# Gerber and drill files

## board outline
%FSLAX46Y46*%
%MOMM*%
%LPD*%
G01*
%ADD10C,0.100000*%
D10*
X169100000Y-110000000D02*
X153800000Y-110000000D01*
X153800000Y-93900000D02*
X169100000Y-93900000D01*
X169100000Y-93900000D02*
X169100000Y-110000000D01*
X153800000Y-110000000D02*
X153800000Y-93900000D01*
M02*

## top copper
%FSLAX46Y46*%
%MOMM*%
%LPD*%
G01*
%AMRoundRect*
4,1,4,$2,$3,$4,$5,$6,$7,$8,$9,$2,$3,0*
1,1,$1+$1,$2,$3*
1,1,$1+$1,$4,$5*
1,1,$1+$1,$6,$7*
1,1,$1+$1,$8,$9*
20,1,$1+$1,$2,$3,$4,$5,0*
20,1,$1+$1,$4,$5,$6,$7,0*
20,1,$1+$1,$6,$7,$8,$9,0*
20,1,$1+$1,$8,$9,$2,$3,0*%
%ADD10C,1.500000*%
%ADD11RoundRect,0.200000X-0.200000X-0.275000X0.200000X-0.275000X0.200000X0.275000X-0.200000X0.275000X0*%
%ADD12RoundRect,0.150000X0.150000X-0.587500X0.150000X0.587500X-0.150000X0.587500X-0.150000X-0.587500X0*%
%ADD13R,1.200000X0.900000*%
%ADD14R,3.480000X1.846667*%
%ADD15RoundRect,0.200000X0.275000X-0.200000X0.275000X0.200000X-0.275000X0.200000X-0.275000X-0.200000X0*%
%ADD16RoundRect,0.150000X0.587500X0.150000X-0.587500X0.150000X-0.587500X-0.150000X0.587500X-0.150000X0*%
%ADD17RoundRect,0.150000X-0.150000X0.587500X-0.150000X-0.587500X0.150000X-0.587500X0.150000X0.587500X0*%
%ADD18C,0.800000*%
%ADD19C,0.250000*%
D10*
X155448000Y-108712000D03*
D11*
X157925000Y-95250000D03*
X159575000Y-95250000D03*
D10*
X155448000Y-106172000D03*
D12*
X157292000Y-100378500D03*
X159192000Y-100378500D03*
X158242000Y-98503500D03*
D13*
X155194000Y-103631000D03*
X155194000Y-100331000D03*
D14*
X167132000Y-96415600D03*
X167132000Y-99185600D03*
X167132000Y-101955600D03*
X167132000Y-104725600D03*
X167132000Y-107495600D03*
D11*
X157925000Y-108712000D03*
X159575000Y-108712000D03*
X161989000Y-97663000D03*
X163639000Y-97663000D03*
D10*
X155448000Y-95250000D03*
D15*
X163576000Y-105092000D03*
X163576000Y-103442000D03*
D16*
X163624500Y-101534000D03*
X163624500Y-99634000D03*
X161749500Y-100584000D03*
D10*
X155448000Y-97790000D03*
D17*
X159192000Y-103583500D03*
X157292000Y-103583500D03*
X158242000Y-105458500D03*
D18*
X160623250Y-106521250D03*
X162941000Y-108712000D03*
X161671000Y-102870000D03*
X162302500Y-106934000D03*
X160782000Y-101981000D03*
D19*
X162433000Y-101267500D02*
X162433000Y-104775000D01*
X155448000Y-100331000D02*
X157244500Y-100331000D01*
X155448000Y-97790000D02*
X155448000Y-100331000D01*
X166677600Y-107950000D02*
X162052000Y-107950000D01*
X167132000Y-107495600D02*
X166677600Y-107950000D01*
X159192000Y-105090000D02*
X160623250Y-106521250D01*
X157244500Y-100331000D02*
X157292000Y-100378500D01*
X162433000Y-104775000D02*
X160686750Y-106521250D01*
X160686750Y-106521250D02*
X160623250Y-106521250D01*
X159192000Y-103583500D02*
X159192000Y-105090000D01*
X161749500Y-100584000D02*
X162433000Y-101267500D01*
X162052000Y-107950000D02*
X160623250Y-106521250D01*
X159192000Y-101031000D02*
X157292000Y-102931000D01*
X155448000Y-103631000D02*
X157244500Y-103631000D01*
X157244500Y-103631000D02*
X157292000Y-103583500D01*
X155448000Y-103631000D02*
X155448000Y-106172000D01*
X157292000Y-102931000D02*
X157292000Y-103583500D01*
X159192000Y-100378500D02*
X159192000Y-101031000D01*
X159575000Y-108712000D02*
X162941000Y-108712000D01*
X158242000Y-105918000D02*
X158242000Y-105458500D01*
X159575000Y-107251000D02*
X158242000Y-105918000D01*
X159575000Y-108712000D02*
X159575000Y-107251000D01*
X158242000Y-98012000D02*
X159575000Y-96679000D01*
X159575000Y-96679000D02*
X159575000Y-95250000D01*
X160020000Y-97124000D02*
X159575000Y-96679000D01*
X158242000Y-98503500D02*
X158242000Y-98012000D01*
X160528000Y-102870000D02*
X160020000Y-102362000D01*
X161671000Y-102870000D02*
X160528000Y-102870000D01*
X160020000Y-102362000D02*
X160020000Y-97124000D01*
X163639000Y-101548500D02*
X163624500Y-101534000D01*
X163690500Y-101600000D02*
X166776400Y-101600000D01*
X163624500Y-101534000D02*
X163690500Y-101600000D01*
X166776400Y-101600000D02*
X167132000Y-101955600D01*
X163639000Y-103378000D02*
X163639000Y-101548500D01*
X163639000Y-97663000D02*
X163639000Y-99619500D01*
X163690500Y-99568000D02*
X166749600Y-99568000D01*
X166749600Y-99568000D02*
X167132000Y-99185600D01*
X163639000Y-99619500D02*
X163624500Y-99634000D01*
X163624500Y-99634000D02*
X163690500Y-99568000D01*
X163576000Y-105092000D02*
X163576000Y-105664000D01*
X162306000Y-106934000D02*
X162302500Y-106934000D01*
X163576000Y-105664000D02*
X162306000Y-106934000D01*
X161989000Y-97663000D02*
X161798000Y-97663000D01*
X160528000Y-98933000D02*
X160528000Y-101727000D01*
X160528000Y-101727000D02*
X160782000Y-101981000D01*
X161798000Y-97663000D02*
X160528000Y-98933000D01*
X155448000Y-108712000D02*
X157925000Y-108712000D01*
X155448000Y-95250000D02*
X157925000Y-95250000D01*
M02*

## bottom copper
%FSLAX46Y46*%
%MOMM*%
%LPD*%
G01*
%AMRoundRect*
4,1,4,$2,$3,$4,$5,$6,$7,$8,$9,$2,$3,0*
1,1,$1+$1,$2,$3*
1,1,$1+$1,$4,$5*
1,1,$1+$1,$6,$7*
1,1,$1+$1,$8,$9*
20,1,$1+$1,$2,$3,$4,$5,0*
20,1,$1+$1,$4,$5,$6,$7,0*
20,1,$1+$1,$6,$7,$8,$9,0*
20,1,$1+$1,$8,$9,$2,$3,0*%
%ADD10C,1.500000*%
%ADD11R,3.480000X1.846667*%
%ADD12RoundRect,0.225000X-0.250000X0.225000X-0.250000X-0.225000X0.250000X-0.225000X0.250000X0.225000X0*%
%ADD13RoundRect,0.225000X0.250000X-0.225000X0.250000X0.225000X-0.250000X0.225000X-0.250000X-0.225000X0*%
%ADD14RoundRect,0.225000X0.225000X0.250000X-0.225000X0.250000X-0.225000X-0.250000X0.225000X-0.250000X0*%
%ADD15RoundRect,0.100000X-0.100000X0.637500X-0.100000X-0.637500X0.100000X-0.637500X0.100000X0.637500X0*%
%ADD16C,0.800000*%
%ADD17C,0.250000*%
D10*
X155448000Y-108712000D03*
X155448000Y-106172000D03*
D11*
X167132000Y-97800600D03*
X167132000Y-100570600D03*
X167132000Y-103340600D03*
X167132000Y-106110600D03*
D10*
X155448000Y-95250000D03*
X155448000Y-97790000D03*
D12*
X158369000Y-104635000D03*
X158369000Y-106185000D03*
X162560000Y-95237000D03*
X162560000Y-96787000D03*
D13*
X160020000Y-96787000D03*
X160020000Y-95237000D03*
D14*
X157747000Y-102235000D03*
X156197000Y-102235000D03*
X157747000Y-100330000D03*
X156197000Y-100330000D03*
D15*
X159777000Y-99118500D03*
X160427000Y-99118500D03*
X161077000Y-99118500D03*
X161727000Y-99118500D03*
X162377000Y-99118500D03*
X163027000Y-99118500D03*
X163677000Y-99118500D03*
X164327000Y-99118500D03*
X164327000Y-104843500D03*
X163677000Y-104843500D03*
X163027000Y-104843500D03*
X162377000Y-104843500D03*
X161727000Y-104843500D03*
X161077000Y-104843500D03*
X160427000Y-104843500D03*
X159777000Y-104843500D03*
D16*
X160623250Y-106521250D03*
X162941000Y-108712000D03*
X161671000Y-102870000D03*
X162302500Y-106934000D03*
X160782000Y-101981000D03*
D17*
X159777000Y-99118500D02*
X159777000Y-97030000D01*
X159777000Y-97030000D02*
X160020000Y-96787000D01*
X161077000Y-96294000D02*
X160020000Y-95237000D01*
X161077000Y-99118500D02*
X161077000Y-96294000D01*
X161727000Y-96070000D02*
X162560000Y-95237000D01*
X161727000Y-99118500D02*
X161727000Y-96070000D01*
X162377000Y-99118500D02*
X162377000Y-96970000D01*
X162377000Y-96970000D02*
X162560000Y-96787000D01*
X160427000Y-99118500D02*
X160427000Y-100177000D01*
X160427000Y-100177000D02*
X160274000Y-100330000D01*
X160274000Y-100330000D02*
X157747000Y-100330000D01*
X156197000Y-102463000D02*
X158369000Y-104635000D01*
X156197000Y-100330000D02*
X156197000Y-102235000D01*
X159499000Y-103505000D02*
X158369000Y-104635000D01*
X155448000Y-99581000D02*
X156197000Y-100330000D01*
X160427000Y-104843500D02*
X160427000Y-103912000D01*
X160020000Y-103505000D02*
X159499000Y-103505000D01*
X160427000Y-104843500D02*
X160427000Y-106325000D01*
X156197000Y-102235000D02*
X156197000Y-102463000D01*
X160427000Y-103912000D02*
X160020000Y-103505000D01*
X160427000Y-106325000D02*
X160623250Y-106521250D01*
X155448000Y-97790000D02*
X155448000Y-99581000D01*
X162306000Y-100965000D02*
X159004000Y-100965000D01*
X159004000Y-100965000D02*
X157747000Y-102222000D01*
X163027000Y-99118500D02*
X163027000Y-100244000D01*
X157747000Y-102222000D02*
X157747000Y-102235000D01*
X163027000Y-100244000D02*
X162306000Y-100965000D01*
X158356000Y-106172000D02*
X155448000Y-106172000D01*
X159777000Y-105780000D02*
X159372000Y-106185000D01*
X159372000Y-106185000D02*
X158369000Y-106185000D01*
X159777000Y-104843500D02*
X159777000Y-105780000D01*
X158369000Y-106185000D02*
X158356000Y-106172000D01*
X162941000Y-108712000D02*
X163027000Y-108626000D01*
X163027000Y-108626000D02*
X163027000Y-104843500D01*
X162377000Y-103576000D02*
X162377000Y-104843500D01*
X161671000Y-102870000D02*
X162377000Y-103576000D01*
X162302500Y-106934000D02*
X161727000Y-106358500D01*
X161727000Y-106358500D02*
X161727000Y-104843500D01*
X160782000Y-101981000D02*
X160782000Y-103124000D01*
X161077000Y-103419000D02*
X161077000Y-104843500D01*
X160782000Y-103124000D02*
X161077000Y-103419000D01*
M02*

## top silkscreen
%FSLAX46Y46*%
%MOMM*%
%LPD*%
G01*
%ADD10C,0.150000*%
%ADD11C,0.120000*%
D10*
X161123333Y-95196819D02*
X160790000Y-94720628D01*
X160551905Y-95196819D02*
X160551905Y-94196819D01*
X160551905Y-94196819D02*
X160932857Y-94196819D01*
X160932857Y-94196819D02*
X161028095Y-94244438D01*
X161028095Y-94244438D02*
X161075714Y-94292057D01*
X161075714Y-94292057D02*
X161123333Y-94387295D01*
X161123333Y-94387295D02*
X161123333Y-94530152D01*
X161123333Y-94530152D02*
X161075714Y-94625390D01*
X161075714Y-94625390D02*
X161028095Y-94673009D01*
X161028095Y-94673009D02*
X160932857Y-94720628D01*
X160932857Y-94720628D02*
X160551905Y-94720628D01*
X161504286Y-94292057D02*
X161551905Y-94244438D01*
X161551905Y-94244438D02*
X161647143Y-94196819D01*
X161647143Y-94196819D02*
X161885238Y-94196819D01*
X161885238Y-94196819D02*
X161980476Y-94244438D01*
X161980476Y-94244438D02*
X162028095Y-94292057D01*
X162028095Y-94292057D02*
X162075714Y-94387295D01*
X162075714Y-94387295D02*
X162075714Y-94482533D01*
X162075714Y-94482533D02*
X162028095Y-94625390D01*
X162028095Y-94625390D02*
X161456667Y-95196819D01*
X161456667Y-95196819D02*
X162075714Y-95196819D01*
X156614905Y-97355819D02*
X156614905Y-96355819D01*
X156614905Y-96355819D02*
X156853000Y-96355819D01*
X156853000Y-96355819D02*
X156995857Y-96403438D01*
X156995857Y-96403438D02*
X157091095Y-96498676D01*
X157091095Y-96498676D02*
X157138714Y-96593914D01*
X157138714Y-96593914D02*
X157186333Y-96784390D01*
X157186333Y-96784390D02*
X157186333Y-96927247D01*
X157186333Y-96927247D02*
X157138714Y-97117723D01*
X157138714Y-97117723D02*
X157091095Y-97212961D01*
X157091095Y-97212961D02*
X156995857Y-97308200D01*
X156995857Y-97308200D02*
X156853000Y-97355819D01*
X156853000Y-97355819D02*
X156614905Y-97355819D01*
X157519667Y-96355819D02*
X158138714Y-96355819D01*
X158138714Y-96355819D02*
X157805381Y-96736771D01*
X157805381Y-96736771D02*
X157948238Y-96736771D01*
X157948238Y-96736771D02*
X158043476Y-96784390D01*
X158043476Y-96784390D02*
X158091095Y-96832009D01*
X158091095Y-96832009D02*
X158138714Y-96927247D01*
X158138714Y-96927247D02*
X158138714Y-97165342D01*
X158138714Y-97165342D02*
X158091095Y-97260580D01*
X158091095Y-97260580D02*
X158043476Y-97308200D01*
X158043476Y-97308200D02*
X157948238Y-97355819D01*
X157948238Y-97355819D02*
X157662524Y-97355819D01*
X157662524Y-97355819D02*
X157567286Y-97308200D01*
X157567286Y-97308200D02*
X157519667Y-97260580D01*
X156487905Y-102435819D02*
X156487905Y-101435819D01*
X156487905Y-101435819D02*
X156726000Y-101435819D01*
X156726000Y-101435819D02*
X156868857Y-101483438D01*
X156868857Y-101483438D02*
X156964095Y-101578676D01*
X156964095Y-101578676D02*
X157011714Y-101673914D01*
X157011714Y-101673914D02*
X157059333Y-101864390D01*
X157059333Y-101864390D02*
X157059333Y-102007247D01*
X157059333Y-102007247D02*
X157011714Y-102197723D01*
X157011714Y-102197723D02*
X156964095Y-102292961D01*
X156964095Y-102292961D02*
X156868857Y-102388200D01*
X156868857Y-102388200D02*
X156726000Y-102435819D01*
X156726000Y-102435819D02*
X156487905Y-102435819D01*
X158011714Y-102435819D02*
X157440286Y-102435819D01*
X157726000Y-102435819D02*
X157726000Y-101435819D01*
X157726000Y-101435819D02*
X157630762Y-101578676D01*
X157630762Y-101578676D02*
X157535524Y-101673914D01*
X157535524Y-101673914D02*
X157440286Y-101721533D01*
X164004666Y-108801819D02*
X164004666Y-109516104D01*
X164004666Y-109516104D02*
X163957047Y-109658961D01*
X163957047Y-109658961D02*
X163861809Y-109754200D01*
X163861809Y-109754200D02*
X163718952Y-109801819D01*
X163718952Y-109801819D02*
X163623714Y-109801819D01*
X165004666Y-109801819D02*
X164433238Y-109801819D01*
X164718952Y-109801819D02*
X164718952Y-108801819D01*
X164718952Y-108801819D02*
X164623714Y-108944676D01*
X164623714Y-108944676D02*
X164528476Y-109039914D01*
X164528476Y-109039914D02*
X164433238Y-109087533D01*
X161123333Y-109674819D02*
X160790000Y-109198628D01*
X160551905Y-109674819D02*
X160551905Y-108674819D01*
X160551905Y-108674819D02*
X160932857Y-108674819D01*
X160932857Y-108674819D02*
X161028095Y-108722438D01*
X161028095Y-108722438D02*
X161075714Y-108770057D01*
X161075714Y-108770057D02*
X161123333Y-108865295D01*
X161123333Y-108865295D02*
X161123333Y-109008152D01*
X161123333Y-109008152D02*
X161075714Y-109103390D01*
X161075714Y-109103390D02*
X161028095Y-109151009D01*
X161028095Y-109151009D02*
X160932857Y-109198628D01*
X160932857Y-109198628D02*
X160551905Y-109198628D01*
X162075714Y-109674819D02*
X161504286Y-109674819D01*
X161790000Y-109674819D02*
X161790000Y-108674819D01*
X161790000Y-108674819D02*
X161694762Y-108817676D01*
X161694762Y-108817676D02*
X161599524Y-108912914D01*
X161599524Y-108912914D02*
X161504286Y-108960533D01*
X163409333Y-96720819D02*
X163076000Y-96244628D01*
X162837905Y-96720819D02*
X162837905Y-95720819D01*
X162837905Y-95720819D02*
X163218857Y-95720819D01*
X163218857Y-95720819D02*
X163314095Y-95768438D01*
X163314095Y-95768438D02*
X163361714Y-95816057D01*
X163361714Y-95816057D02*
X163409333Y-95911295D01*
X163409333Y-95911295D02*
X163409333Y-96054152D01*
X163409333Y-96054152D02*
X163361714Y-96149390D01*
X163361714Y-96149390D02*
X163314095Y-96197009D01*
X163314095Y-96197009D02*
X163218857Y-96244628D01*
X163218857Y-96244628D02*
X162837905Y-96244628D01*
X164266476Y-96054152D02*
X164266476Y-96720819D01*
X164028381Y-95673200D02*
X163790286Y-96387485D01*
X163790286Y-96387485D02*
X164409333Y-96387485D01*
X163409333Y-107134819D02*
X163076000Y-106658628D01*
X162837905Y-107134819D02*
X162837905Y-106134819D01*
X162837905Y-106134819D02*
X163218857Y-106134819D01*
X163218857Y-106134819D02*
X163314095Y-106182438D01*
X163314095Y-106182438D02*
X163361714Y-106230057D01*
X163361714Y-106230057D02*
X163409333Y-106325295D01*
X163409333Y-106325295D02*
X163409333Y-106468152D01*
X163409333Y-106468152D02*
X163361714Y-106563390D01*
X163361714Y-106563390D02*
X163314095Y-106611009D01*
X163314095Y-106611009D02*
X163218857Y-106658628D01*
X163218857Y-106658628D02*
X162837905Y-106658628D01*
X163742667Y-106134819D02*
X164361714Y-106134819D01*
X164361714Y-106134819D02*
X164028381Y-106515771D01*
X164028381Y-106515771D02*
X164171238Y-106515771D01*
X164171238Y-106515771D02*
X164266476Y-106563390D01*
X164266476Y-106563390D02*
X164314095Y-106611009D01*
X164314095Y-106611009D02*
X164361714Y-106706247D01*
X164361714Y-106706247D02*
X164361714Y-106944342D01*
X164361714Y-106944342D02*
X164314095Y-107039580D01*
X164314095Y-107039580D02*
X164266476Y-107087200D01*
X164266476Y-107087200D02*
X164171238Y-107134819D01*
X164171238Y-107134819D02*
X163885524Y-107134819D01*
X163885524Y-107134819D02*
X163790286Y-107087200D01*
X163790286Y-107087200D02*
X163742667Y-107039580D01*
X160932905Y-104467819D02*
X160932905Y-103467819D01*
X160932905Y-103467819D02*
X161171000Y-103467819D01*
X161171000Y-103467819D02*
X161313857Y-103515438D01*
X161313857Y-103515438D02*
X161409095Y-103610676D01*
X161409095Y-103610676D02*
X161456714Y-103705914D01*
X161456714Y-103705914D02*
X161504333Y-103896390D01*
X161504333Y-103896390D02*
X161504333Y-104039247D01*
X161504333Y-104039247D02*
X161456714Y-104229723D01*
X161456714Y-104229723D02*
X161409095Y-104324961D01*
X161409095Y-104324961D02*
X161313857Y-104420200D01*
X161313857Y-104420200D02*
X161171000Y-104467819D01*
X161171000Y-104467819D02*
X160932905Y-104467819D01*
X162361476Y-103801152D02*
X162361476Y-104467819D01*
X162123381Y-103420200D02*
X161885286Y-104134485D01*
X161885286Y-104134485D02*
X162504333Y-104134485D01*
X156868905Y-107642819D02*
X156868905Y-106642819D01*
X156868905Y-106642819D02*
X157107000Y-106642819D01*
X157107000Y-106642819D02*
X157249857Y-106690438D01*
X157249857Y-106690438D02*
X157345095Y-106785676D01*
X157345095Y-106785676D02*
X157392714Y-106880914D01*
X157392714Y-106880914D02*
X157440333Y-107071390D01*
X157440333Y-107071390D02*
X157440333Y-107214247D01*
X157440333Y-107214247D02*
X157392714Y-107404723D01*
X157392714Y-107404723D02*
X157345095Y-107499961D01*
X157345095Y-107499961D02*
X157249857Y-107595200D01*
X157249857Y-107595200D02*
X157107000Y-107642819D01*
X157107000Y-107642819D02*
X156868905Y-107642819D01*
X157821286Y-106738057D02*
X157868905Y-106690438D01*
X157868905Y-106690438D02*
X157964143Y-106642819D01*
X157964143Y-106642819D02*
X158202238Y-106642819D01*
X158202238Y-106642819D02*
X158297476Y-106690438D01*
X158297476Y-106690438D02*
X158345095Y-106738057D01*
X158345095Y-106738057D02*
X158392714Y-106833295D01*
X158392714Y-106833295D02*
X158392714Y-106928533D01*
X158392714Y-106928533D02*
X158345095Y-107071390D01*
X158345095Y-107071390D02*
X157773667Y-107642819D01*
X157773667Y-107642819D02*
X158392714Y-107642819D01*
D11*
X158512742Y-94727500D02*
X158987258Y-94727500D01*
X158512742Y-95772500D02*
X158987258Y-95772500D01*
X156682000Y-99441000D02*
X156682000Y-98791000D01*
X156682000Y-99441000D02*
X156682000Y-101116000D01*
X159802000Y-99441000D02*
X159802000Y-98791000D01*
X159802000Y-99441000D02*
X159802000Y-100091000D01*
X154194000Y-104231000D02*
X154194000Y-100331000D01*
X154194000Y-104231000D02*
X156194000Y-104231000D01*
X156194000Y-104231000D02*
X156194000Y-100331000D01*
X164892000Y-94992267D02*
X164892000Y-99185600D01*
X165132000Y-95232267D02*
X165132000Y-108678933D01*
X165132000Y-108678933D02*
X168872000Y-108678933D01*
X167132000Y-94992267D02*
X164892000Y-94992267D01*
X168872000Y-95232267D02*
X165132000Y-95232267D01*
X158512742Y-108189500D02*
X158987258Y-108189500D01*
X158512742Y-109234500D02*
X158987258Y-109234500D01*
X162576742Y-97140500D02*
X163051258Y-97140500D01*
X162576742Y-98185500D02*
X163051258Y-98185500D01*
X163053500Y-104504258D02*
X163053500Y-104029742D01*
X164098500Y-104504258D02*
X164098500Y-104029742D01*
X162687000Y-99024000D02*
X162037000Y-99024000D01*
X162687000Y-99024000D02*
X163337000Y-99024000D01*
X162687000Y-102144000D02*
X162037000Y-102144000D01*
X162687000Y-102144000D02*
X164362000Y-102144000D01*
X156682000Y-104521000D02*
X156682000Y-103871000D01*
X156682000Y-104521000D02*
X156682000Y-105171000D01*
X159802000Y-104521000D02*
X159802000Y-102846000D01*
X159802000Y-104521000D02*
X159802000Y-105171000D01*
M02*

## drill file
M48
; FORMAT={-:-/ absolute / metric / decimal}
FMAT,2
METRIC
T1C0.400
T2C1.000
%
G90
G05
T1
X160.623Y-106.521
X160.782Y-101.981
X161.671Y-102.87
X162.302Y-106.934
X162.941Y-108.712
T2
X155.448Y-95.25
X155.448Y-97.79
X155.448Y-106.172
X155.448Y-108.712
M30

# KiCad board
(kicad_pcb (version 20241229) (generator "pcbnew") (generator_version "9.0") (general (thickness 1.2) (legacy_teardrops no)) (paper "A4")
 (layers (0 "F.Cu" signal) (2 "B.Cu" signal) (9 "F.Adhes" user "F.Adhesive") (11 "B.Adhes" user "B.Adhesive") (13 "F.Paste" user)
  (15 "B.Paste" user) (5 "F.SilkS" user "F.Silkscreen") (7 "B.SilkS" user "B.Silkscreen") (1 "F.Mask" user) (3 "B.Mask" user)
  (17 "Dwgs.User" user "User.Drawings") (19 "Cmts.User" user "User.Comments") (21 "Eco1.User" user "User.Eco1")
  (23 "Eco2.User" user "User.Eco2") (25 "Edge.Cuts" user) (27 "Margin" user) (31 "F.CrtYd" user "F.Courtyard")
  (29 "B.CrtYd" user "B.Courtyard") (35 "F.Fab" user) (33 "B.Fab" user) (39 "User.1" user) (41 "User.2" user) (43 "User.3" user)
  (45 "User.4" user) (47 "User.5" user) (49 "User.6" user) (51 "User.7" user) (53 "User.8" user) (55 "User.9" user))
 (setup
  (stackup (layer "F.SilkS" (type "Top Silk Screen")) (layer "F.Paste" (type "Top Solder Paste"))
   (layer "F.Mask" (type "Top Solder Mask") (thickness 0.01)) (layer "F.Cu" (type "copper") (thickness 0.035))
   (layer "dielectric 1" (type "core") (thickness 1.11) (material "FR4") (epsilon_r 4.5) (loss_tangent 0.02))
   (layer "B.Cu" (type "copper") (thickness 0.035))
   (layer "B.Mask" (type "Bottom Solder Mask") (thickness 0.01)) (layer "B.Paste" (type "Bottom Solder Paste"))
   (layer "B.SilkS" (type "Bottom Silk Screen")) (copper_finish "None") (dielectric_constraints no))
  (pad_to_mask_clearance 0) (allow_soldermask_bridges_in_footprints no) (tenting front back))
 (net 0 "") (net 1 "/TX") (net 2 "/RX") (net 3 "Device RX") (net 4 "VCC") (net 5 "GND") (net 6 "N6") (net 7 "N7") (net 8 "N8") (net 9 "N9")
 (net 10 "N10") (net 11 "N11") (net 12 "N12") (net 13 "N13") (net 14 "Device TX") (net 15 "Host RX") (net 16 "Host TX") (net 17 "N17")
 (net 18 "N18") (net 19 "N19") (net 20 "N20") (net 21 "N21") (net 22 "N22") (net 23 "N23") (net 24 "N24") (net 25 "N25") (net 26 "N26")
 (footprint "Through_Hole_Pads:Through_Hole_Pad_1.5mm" (layer "F.Cu") (at 155.448 108.712)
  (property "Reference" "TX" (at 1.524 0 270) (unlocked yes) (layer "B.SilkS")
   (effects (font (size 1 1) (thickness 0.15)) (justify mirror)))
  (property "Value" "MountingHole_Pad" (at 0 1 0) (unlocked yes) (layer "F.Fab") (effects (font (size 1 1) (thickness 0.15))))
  (pad "1" thru_hole circle (at 0 0) (size 1.5 1.5) (drill 1) (layers "*.Cu" "*.Mask") (remove_unused_layers no) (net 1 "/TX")))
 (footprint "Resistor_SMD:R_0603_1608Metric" (layer "F.Cu") (at 158.75 95.25)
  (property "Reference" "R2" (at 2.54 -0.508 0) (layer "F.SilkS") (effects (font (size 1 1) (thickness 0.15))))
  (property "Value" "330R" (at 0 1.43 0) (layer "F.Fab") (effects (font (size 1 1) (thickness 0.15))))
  (fp_line (start -0.237258 -0.5225) (end 0.237258 -0.5225) (stroke (width 0.12) (type solid)) (layer "F.SilkS"))
  (fp_line (start -0.237258 0.5225) (end 0.237258 0.5225) (stroke (width 0.12) (type solid)) (layer "F.SilkS"))
  (pad "1" smd roundrect (at -0.825 0) (size 0.8 0.95) (layers "F.Cu" "F.Mask" "F.Paste") (roundrect_rratio 0.25) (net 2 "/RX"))
  (pad "2" smd roundrect (at 0.825 0) (size 0.8 0.95) (layers "F.Cu" "F.Mask" "F.Paste") (roundrect_rratio 0.25) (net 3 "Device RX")))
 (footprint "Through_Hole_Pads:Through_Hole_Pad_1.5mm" (layer "F.Cu") (at 155.448 106.172)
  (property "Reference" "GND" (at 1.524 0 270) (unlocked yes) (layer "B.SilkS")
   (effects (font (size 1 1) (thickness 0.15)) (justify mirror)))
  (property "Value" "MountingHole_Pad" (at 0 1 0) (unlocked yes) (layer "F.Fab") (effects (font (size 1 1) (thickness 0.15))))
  (pad "1" thru_hole circle (at 0 0) (size 1.5 1.5) (drill 1) (layers "*.Cu" "*.Mask") (remove_unused_layers no) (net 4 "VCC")))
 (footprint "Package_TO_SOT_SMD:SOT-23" (layer "F.Cu") (at 158.242 99.441 90)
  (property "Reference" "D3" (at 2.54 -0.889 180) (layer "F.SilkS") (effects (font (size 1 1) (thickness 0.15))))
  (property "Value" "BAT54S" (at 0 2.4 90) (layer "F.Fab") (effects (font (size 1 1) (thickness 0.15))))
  (fp_line (start 0 -1.56) (end 0.65 -1.56) (stroke (width 0.12) (type solid)) (layer "F.SilkS"))
  (fp_line (start 0 -1.56) (end -1.675 -1.56) (stroke (width 0.12) (type solid)) (layer "F.SilkS"))
  (fp_line (start 0 1.56) (end 0.65 1.56) (stroke (width 0.12) (type solid)) (layer "F.SilkS"))
  (fp_line (start 0 1.56) (end -0.65 1.56) (stroke (width 0.12) (type solid)) (layer "F.SilkS"))
  (pad "1" smd roundrect (at -0.9375 -0.95 90) (size 1.475 0.6) (layers "F.Cu" "F.Mask" "F.Paste") (roundrect_rratio 0.25) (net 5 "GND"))
  (pad "2" smd roundrect (at -0.9375 0.95 90) (size 1.475 0.6) (layers "F.Cu" "F.Mask" "F.Paste") (roundrect_rratio 0.25) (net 4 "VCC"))
  (pad "3" smd roundrect (at 0.9375 0 90) (size 1.475 0.6) (layers "F.Cu" "F.Mask" "F.Paste") (roundrect_rratio 0.25) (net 3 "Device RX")))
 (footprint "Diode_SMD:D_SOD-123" (layer "F.Cu") (at 155.194 101.981 90)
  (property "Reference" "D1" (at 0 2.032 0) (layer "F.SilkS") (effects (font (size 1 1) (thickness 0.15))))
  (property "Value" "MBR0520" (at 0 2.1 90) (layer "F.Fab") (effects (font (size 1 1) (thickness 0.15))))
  (fp_line (start -2.25 -1) (end 1.65 -1) (stroke (width 0.12) (type solid)) (layer "F.SilkS"))
  (fp_line (start -2.25 -1) (end -2.25 1) (stroke (width 0.12) (type solid)) (layer "F.SilkS"))
  (fp_line (start -2.25 1) (end 1.65 1) (stroke (width 0.12) (type solid)) (layer "F.SilkS"))
  (pad "1" smd rect (at -1.65 0 90) (size 0.9 1.2) (layers "F.Cu" "F.Mask" "F.Paste") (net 4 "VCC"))
  (pad "2" smd rect (at 1.65 0 90) (size 0.9 1.2) (layers "F.Cu" "F.Mask" "F.Paste") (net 5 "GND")))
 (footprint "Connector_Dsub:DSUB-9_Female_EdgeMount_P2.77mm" (layer "F.Cu") (at 167.132 101.9556 90)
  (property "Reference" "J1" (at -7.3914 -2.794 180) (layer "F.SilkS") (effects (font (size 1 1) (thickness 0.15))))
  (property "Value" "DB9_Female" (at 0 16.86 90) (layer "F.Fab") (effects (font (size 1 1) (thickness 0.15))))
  (fp_line (start 6.963333 -2.24) (end 2.77 -2.24) (stroke (width 0.12) (type solid)) (layer "F.SilkS"))
  (fp_line (start 6.723333 -2) (end -6.723333 -2) (stroke (width 0.12) (type solid)) (layer "F.SilkS"))
  (fp_line (start -6.723333 -2) (end -6.723333 1.74) (stroke (width 0.12) (type solid)) (layer "F.SilkS"))
  (fp_line (start 6.963333 0) (end 6.963333 -2.24) (stroke (width 0.12) (type solid)) (layer "F.SilkS"))
  (fp_line (start 6.723333 1.74) (end 6.723333 -2) (stroke (width 0.12) (type solid)) (layer "F.SilkS"))
  (pad "1" smd rect (at 5.54 0 90) (size 1.846667 3.48) (layers "F.Cu" "F.Mask" "F.Paste") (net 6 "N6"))
  (pad "2" smd rect (at 2.77 0 90) (size 1.846667 3.48) (layers "F.Cu" "F.Mask" "F.Paste") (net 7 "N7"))
  (pad "3" smd rect (at 0 0 90) (size 1.846667 3.48) (layers "F.Cu" "F.Mask" "F.Paste") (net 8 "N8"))
  (pad "4" smd rect (at -2.77 0 90) (size 1.846667 3.48) (layers "F.Cu" "F.Mask" "F.Paste") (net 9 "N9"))
  (pad "5" smd rect (at -5.54 0 90) (size 1.846667 3.48) (layers "F.Cu" "F.Mask" "F.Paste") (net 5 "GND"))
  (pad "6" smd rect (at 4.155 0 90) (size 1.846667 3.48) (layers "B.Cu" "B.Mask" "B.Paste") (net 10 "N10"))
  (pad "7" smd rect (at 1.385 0 90) (size 1.846667 3.48) (layers "B.Cu" "B.Mask" "B.Paste") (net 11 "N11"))
  (pad "8" smd rect (at -1.385 0 90) (size 1.846667 3.48) (layers "B.Cu" "B.Mask" "B.Paste") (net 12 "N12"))
  (pad "9" smd rect (at -4.155 0 90) (size 1.846667 3.48) (layers "B.Cu" "B.Mask" "B.Paste") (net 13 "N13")))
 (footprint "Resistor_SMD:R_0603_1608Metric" (layer "F.Cu") (at 158.75 108.712)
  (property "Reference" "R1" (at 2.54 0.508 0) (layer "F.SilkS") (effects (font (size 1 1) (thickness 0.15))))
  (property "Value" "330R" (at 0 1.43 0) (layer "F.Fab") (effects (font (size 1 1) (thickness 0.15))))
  (fp_line (start -0.237258 -0.5225) (end 0.237258 -0.5225) (stroke (width 0.12) (type solid)) (layer "F.SilkS"))
  (fp_line (start -0.237258 0.5225) (end 0.237258 0.5225) (stroke (width 0.12) (type solid)) (layer "F.SilkS"))
  (pad "1" smd roundrect (at -0.825 0) (size 0.8 0.95) (layers "F.Cu" "F.Mask" "F.Paste") (roundrect_rratio 0.25) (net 1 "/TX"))
  (pad "2" smd roundrect (at 0.825 0) (size 0.8 0.95) (layers "F.Cu" "F.Mask" "F.Paste") (roundrect_rratio 0.25) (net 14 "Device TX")))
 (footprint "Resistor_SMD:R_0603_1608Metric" (layer "F.Cu") (at 162.814 97.663)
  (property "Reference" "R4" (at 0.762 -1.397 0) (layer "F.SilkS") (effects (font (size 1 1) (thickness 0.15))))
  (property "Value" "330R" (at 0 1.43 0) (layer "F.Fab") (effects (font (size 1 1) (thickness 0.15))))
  (fp_line (start -0.237258 -0.5225) (end 0.237258 -0.5225) (stroke (width 0.12) (type solid)) (layer "F.SilkS"))
  (fp_line (start -0.237258 0.5225) (end 0.237258 0.5225) (stroke (width 0.12) (type solid)) (layer "F.SilkS"))
  (pad "1" smd roundrect (at -0.825 0) (size 0.8 0.95) (layers "F.Cu" "F.Mask" "F.Paste") (roundrect_rratio 0.25) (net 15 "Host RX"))
  (pad "2" smd roundrect (at 0.825 0) (size 0.8 0.95) (layers "F.Cu" "F.Mask" "F.Paste") (roundrect_rratio 0.25) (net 7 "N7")))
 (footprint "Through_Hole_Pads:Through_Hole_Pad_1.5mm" (layer "F.Cu") (at 155.448 95.25)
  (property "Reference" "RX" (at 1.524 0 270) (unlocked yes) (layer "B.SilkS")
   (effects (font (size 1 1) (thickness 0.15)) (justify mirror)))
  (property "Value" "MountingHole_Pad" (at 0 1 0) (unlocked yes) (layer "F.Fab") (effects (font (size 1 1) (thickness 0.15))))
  (pad "1" thru_hole circle (at 0 0) (size 1.5 1.5) (drill 1) (layers "*.Cu" "*.Mask") (remove_unused_layers no) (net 2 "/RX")))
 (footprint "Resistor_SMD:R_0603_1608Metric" (layer "F.Cu") (at 163.576 104.267 90)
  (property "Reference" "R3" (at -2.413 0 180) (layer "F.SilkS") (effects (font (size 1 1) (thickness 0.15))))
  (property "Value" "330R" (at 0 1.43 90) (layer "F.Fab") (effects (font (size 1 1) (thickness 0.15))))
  (fp_line (start -0.237258 -0.5225) (end 0.237258 -0.5225) (stroke (width 0.12) (type solid)) (layer "F.SilkS"))
  (fp_line (start -0.237258 0.5225) (end 0.237258 0.5225) (stroke (width 0.12) (type solid)) (layer "F.SilkS"))
  (pad "1" smd roundrect (at -0.825 0 90) (size 0.8 0.95) (layers "F.Cu" "F.Mask" "F.Paste") (roundrect_rratio 0.25) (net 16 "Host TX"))
  (pad "2" smd roundrect (at 0.825 0 90) (size 0.8 0.95) (layers "F.Cu" "F.Mask" "F.Paste") (roundrect_rratio 0.25) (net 8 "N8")))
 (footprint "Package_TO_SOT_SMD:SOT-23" (layer "F.Cu") (at 162.687 100.584 180)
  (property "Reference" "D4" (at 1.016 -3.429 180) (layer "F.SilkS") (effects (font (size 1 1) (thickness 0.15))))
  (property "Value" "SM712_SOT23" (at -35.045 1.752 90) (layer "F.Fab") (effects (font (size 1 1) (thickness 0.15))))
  (fp_line (start 0 1.56) (end 0.65 1.56) (stroke (width 0.12) (type solid)) (layer "F.SilkS"))
  (fp_line (start 0 1.56) (end -0.65 1.56) (stroke (width 0.12) (type solid)) (layer "F.SilkS"))
  (fp_line (start 0 -1.56) (end 0.65 -1.56) (stroke (width 0.12) (type solid)) (layer "F.SilkS"))
  (fp_line (start 0 -1.56) (end -1.675 -1.56) (stroke (width 0.12) (type solid)) (layer "F.SilkS"))
  (pad "1" smd roundrect (at -0.9375 -0.95 180) (size 1.475 0.6) (layers "F.Cu" "F.Mask" "F.Paste") (roundrect_rratio 0.25) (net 8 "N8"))
  (pad "2" smd roundrect (at -0.9375 0.95 180) (size 1.475 0.6) (layers "F.Cu" "F.Mask" "F.Paste") (roundrect_rratio 0.25) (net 7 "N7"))
  (pad "3" smd roundrect (at 0.9375 0 180) (size 1.475 0.6) (layers "F.Cu" "F.Mask" "F.Paste") (roundrect_rratio 0.25) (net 5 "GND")))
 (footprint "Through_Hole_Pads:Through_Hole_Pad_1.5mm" (layer "F.Cu") (at 155.448 97.79 180)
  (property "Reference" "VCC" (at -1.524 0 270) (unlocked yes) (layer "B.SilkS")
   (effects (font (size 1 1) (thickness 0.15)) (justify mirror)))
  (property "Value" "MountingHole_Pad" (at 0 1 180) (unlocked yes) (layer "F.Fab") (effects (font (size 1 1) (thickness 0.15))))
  (pad "1" thru_hole circle (at 0 0 180) (size 1.5 1.5) (drill 1) (layers "*.Cu" "*.Mask") (remove_unused_layers no) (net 5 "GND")))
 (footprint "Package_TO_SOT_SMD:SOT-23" (layer "F.Cu") (at 158.242 104.521 -90)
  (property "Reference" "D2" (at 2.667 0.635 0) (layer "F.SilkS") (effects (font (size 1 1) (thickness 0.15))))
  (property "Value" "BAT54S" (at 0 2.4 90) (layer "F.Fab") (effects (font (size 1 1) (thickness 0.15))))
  (fp_line (start 0 1.56) (end -0.65 1.56) (stroke (width 0.12) (type solid)) (layer "F.SilkS"))
  (fp_line (start 0 1.56) (end 0.65 1.56) (stroke (width 0.12) (type solid)) (layer "F.SilkS"))
  (fp_line (start 0 -1.56) (end -1.675 -1.56) (stroke (width 0.12) (type solid)) (layer "F.SilkS"))
  (fp_line (start 0 -1.56) (end 0.65 -1.56) (stroke (width 0.12) (type solid)) (layer "F.SilkS"))
  (pad "1" smd roundrect (at -0.9375 -0.95 270) (size 1.475 0.6) (layers "F.Cu" "F.Mask" "F.Paste") (roundrect_rratio 0.25) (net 5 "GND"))
  (pad "2" smd roundrect (at -0.9375 0.95 270) (size 1.475 0.6) (layers "F.Cu" "F.Mask" "F.Paste") (roundrect_rratio 0.25) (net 4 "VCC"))
  (pad "3" smd roundrect (at 0.9375 0 270) (size 1.475 0.6) (layers "F.Cu" "F.Mask" "F.Paste") (roundrect_rratio 0.25) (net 14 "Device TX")))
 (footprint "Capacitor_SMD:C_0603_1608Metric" (layer "B.Cu") (at 158.369 105.41 -90)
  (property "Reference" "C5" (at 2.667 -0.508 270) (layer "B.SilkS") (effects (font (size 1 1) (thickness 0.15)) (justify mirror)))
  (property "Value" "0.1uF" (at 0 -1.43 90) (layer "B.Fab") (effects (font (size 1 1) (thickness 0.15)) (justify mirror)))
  (pad "1" smd roundrect (at -0.775 0 270) (size 0.9 0.95) (layers "B.Cu" "B.Mask" "B.Paste") (roundrect_rratio 0.25) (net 5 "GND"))
  (pad "2" smd roundrect (at 0.775 0 270) (size 0.9 0.95) (layers "B.Cu" "B.Mask" "B.Paste") (roundrect_rratio 0.25) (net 4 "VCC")))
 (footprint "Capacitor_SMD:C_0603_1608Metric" (layer "B.Cu") (at 162.56 96.012 -90)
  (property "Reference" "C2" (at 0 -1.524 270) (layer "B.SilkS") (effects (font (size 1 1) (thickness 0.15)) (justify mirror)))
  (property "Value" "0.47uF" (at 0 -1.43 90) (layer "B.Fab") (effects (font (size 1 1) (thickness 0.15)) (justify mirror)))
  (pad "1" smd roundrect (at -0.775 0 270) (size 0.9 0.95) (layers "B.Cu" "B.Mask" "B.Paste") (roundrect_rratio 0.25) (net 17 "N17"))
  (pad "2" smd roundrect (at 0.775 0 270) (size 0.9 0.95) (layers "B.Cu" "B.Mask" "B.Paste") (roundrect_rratio 0.25) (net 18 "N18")))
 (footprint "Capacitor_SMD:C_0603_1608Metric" (layer "B.Cu") (at 160.02 96.012 90)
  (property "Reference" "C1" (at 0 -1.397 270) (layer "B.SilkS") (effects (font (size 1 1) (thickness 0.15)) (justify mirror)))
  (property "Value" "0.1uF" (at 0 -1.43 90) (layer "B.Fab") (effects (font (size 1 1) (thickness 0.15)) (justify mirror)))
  (pad "1" smd roundrect (at -0.775 0 90) (size 0.9 0.95) (layers "B.Cu" "B.Mask" "B.Paste") (roundrect_rratio 0.25) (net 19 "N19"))
  (pad "2" smd roundrect (at 0.775 0 90) (size 0.9 0.95) (layers "B.Cu" "B.Mask" "B.Paste") (roundrect_rratio 0.25) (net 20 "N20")))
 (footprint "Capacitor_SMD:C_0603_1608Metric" (layer "B.Cu") (at 156.972 102.235 180)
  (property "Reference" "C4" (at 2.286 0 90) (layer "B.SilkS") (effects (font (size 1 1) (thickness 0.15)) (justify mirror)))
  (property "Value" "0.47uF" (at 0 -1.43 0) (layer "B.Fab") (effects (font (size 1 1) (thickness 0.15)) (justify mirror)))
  (pad "1" smd roundrect (at -0.775 0 180) (size 0.9 0.95) (layers "B.Cu" "B.Mask" "B.Paste") (roundrect_rratio 0.25) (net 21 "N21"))
  (pad "2" smd roundrect (at 0.775 0 180) (size 0.9 0.95) (layers "B.Cu" "B.Mask" "B.Paste") (roundrect_rratio 0.25) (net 5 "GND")))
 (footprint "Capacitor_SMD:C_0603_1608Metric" (layer "B.Cu") (at 156.972 100.33 180)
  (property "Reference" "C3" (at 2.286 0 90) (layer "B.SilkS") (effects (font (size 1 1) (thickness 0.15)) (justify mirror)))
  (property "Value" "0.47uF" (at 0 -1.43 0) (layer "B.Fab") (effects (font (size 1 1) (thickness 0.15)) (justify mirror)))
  (pad "1" smd roundrect (at -0.775 0 180) (size 0.9 0.95) (layers "B.Cu" "B.Mask" "B.Paste") (roundrect_rratio 0.25) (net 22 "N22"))
  (pad "2" smd roundrect (at 0.775 0 180) (size 0.9 0.95) (layers "B.Cu" "B.Mask" "B.Paste") (roundrect_rratio 0.25) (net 5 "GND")))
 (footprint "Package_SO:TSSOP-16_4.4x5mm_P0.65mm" (layer "B.Cu") (at 162.052 101.981 -90)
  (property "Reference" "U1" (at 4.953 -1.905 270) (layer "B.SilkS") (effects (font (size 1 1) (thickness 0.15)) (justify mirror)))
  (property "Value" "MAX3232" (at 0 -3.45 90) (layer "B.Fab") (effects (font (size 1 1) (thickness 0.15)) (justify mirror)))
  (pad "1" smd roundrect (at -2.8625 2.275 270) (size 1.475 0.4) (layers "B.Cu" "B.Mask" "B.Paste") (roundrect_rratio 0.25) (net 19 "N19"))
  (pad "2" smd roundrect (at -2.8625 1.625 270) (size 1.475 0.4) (layers "B.Cu" "B.Mask" "B.Paste") (roundrect_rratio 0.25) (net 22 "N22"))
  (pad "3" smd roundrect (at -2.8625 0.975 270) (size 1.475 0.4) (layers "B.Cu" "B.Mask" "B.Paste") (roundrect_rratio 0.25) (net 20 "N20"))
  (pad "4" smd roundrect (at -2.8625 0.325 270) (size 1.475 0.4) (layers "B.Cu" "B.Mask" "B.Paste") (roundrect_rratio 0.25) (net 17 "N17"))
  (pad "5" smd roundrect (at -2.8625 -0.325 270) (size 1.475 0.4) (layers "B.Cu" "B.Mask" "B.Paste") (roundrect_rratio 0.25) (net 18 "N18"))
  (pad "6" smd roundrect (at -2.8625 -0.975 270) (size 1.475 0.4) (layers "B.Cu" "B.Mask" "B.Paste") (roundrect_rratio 0.25) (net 21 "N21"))
  (pad "7" smd roundrect (at -2.8625 -1.625 270) (size 1.475 0.4) (layers "B.Cu" "B.Mask" "B.Paste") (roundrect_rratio 0.25) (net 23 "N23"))
  (pad "8" smd roundrect (at -2.8625 -2.275 270) (size 1.475 0.4) (layers "B.Cu" "B.Mask" "B.Paste") (roundrect_rratio 0.25) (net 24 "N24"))
  (pad "9" smd roundrect (at 2.8625 -2.275 270) (size 1.475 0.4) (layers "B.Cu" "B.Mask" "B.Paste") (roundrect_rratio 0.25) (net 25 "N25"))
  (pad "10" smd roundrect (at 2.8625 -1.625 270) (size 1.475 0.4) (layers "B.Cu" "B.Mask" "B.Paste") (roundrect_rratio 0.25) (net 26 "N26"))
  (pad "11" smd roundrect (at 2.8625 -0.975 270) (size 1.475 0.4) (layers "B.Cu" "B.Mask" "B.Paste") (roundrect_rratio 0.25)
   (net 14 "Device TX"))
  (pad "12" smd roundrect (at 2.8625 -0.325 270) (size 1.475 0.4) (layers "B.Cu" "B.Mask" "B.Paste") (roundrect_rratio 0.25)
   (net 3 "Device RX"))
  (pad "13" smd roundrect (at 2.8625 0.325 270) (size 1.475 0.4) (layers "B.Cu" "B.Mask" "B.Paste") (roundrect_rratio 0.25)
   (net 16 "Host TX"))
  (pad "14" smd roundrect (at 2.8625 0.975 270) (size 1.475 0.4) (layers "B.Cu" "B.Mask" "B.Paste") (roundrect_rratio 0.25)
   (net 15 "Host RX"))
  (pad "15" smd roundrect (at 2.8625 1.625 270) (size 1.475 0.4) (layers "B.Cu" "B.Mask" "B.Paste") (roundrect_rratio 0.25) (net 5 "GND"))
  (pad "16" smd roundrect (at 2.8625 2.275 270) (size 1.475 0.4) (layers "B.Cu" "B.Mask" "B.Paste") (roundrect_rratio 0.25) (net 4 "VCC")))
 (gr_line (start 169.1 110) (end 153.8 110) (stroke (width 0.1) (type solid)) (layer "Edge.Cuts"))
 (gr_line (start 153.8 93.9) (end 169.1 93.9) (stroke (width 0.1) (type solid)) (layer "Edge.Cuts"))
 (gr_line (start 169.1 93.9) (end 169.1 110) (stroke (width 0.1) (type solid)) (layer "Edge.Cuts"))
 (gr_line (start 153.8 110) (end 153.8 93.9) (stroke (width 0.1) (type solid)) (layer "Edge.Cuts"))
 (segment (start 159.777 99.1185) (end 159.777 97.03) (width 0.25) (layer "B.Cu") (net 19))
 (segment (start 159.777 97.03) (end 160.02 96.787) (width 0.25) (layer "B.Cu") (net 19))
 (segment (start 161.077 96.294) (end 160.02 95.237) (width 0.25) (layer "B.Cu") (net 20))
 (segment (start 161.077 99.1185) (end 161.077 96.294) (width 0.25) (layer "B.Cu") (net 20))
 (segment (start 161.727 96.07) (end 162.56 95.237) (width 0.25) (layer "B.Cu") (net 17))
 (segment (start 161.727 99.1185) (end 161.727 96.07) (width 0.25) (layer "B.Cu") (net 17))
 (segment (start 162.377 99.1185) (end 162.377 96.97) (width 0.25) (layer "B.Cu") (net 18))
 (segment (start 162.377 96.97) (end 162.56 96.787) (width 0.25) (layer "B.Cu") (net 18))
 (segment (start 160.427 99.1185) (end 160.427 100.177) (width 0.25) (layer "B.Cu") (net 22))
 (segment (start 160.427 100.177) (end 160.274 100.33) (width 0.25) (layer "B.Cu") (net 22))
 (segment (start 160.274 100.33) (end 157.747 100.33) (width 0.25) (layer "B.Cu") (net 22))
 (segment (start 162.433 101.2675) (end 162.433 104.775) (width 0.25) (layer "F.Cu") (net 5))
 (segment (start 155.448 100.331) (end 157.2445 100.331) (width 0.25) (layer "F.Cu") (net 5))
 (segment (start 155.448 97.79) (end 155.448 100.331) (width 0.25) (layer "F.Cu") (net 5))
 (segment (start 166.6776 107.95) (end 162.052 107.95) (width 0.25) (layer "F.Cu") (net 5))
 (segment (start 167.132 107.4956) (end 166.6776 107.95) (width 0.25) (layer "F.Cu") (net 5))
 (segment (start 159.192 105.09) (end 160.62325 106.52125) (width 0.25) (layer "F.Cu") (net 5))
 (segment (start 157.2445 100.331) (end 157.292 100.3785) (width 0.25) (layer "F.Cu") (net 5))
 (segment (start 162.433 104.775) (end 160.68675 106.52125) (width 0.25) (layer "F.Cu") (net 5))
 (segment (start 160.68675 106.52125) (end 160.62325 106.52125) (width 0.25) (layer "F.Cu") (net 5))
 (segment (start 159.192 103.5835) (end 159.192 105.09) (width 0.25) (layer "F.Cu") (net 5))
 (segment (start 161.7495 100.584) (end 162.433 101.2675) (width 0.25) (layer "F.Cu") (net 5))
 (segment (start 162.052 107.95) (end 160.62325 106.52125) (width 0.25) (layer "F.Cu") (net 5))
 (via (at 160.62325 106.52125) (size 0.8) (drill 0.4) (layers "F.Cu" "B.Cu") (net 5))
 (segment (start 156.197 102.463) (end 158.369 104.635) (width 0.25) (layer "B.Cu") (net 5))
 (segment (start 156.197 100.33) (end 156.197 102.235) (width 0.25) (layer "B.Cu") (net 5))
 (segment (start 159.499 103.505) (end 158.369 104.635) (width 0.25) (layer "B.Cu") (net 5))
 (segment (start 155.448 99.581) (end 156.197 100.33) (width 0.25) (layer "B.Cu") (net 5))
 (segment (start 160.427 104.8435) (end 160.427 103.912) (width 0.25) (layer "B.Cu") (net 5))
 (segment (start 160.02 103.505) (end 159.499 103.505) (width 0.25) (layer "B.Cu") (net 5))
 (segment (start 160.427 104.8435) (end 160.427 106.325) (width 0.25) (layer "B.Cu") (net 5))
 (segment (start 156.197 102.235) (end 156.197 102.463) (width 0.25) (layer "B.Cu") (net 5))
 (segment (start 160.427 103.912) (end 160.02 103.505) (width 0.25) (layer "B.Cu") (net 5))
 (segment (start 160.427 106.325) (end 160.62325 106.52125) (width 0.25) (layer "B.Cu") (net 5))
 (segment (start 155.448 97.79) (end 155.448 99.581) (width 0.25) (layer "B.Cu") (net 5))
 (segment (start 162.306 100.965) (end 159.004 100.965) (width 0.25) (layer "B.Cu") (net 21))
 (segment (start 159.004 100.965) (end 157.747 102.222) (width 0.25) (layer "B.Cu") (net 21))
 (segment (start 163.027 99.1185) (end 163.027 100.244) (width 0.25) (layer "B.Cu") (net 21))
 (segment (start 157.747 102.222) (end 157.747 102.235) (width 0.25) (layer "B.Cu") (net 21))
 (segment (start 163.027 100.244) (end 162.306 100.965) (width 0.25) (layer "B.Cu") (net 21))
 (segment (start 159.192 101.031) (end 157.292 102.931) (width 0.25) (layer "F.Cu") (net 4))
 (segment (start 155.448 103.631) (end 157.2445 103.631) (width 0.25) (layer "F.Cu") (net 4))
 (segment (start 157.2445 103.631) (end 157.292 103.5835) (width 0.25) (layer "F.Cu") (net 4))
 (segment (start 155.448 103.631) (end 155.448 106.172) (width 0.25) (layer "F.Cu") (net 4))
 (segment (start 157.292 102.931) (end 157.292 103.5835) (width 0.25) (layer "F.Cu") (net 4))
 (segment (start 159.192 100.3785) (end 159.192 101.031) (width 0.25) (layer "F.Cu") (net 4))
 (segment (start 158.356 106.172) (end 155.448 106.172) (width 0.25) (layer "B.Cu") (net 4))
 (segment (start 159.777 105.78) (end 159.372 106.185) (width 0.25) (layer "B.Cu") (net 4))
 (segment (start 159.372 106.185) (end 158.369 106.185) (width 0.25) (layer "B.Cu") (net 4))
 (segment (start 159.777 104.8435) (end 159.777 105.78) (width 0.25) (layer "B.Cu") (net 4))
 (segment (start 158.369 106.185) (end 158.356 106.172) (width 0.25) (layer "B.Cu") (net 4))
 (segment (start 159.575 108.712) (end 162.941 108.712) (width 0.25) (layer "F.Cu") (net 14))
 (segment (start 158.242 105.918) (end 158.242 105.4585) (width 0.25) (layer "F.Cu") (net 14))
 (segment (start 159.575 107.251) (end 158.242 105.918) (width 0.25) (layer "F.Cu") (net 14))
 (segment (start 159.575 108.712) (end 159.575 107.251) (width 0.25) (layer "F.Cu") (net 14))
 (via (at 162.941 108.712) (size 0.8) (drill 0.4) (layers "F.Cu" "B.Cu") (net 14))
 (segment (start 162.941 108.712) (end 163.027 108.626) (width 0.25) (layer "B.Cu") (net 14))
 (segment (start 163.027 108.626) (end 163.027 104.8435) (width 0.25) (layer "B.Cu") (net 14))
 (segment (start 158.242 98.012) (end 159.575 96.679) (width 0.25) (layer "F.Cu") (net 3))
 (segment (start 159.575 96.679) (end 159.575 95.25) (width 0.25) (layer "F.Cu") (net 3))
 (segment (start 160.02 97.124) (end 159.575 96.679) (width 0.25) (layer "F.Cu") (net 3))
 (segment (start 158.242 98.5035) (end 158.242 98.012) (width 0.25) (layer "F.Cu") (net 3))
 (segment (start 160.528 102.87) (end 160.02 102.362) (width 0.25) (layer "F.Cu") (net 3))
 (segment (start 161.671 102.87) (end 160.528 102.87) (width 0.25) (layer "F.Cu") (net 3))
 (segment (start 160.02 102.362) (end 160.02 97.124) (width 0.25) (layer "F.Cu") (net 3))
 (via (at 161.671 102.87) (size 0.8) (drill 0.4) (layers "F.Cu" "B.Cu") (free yes) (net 3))
 (segment (start 162.377 103.576) (end 162.377 104.8435) (width 0.25) (layer "B.Cu") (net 3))
 (segment (start 161.671 102.87) (end 162.377 103.576) (width 0.25) (layer "B.Cu") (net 3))
 (segment (start 163.639 101.5485) (end 163.6245 101.534) (width 0.25) (layer "F.Cu") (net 8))
 (segment (start 163.6905 101.6) (end 166.7764 101.6) (width 0.25) (layer "F.Cu") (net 8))
 (segment (start 163.6245 101.534) (end 163.6905 101.6) (width 0.25) (layer "F.Cu") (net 8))
 (segment (start 166.7764 101.6) (end 167.132 101.9556) (width 0.25) (layer "F.Cu") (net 8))
 (segment (start 163.639 103.378) (end 163.639 101.5485) (width 0.25) (layer "F.Cu") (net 8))
 (segment (start 163.639 97.663) (end 163.639 99.6195) (width 0.25) (layer "F.Cu") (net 7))
 (segment (start 163.6905 99.568) (end 166.7496 99.568) (width 0.25) (layer "F.Cu") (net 7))
 (segment (start 166.7496 99.568) (end 167.132 99.1856) (width 0.25) (layer "F.Cu") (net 7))
 (segment (start 163.639 99.6195) (end 163.6245 99.634) (width 0.25) (layer "F.Cu") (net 7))
 (segment (start 163.6245 99.634) (end 163.6905 99.568) (width 0.25) (layer "F.Cu") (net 7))
 (segment (start 163.576 105.092) (end 163.576 105.664) (width 0.25) (layer "F.Cu") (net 16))
 (segment (start 162.306 106.934) (end 162.3025 106.934) (width 0.25) (layer "F.Cu") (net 16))
 (segment (start 163.576 105.664) (end 162.306 106.934) (width 0.25) (layer "F.Cu") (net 16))
 (via (at 162.3025 106.934) (size 0.8) (drill 0.4) (layers "F.Cu" "B.Cu") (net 16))
 (segment (start 162.3025 106.934) (end 161.727 106.3585) (width 0.25) (layer "B.Cu") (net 16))
 (segment (start 161.727 106.3585) (end 161.727 104.8435) (width 0.25) (layer "B.Cu") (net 16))
 (segment (start 161.989 97.663) (end 161.798 97.663) (width 0.25) (layer "F.Cu") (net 15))
 (segment (start 160.528 98.933) (end 160.528 101.727) (width 0.25) (layer "F.Cu") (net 15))
 (segment (start 160.528 101.727) (end 160.782 101.981) (width 0.25) (layer "F.Cu") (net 15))
 (segment (start 161.798 97.663) (end 160.528 98.933) (width 0.25) (layer "F.Cu") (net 15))
 (via (at 160.782 101.981) (size 0.8) (drill 0.4) (layers "F.Cu" "B.Cu") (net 15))
 (segment (start 160.782 101.981) (end 160.782 103.124) (width 0.25) (layer "B.Cu") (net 15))
 (segment (start 161.077 103.419) (end 161.077 104.8435) (width 0.25) (layer "B.Cu") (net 15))
 (segment (start 160.782 103.124) (end 161.077 103.419) (width 0.25) (layer "B.Cu") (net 15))
 (segment (start 155.448 108.712) (end 157.925 108.712) (width 0.25) (layer "F.Cu") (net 1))
 (segment (start 155.448 95.25) (end 157.925 95.25) (width 0.25) (layer "F.Cu") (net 2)))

